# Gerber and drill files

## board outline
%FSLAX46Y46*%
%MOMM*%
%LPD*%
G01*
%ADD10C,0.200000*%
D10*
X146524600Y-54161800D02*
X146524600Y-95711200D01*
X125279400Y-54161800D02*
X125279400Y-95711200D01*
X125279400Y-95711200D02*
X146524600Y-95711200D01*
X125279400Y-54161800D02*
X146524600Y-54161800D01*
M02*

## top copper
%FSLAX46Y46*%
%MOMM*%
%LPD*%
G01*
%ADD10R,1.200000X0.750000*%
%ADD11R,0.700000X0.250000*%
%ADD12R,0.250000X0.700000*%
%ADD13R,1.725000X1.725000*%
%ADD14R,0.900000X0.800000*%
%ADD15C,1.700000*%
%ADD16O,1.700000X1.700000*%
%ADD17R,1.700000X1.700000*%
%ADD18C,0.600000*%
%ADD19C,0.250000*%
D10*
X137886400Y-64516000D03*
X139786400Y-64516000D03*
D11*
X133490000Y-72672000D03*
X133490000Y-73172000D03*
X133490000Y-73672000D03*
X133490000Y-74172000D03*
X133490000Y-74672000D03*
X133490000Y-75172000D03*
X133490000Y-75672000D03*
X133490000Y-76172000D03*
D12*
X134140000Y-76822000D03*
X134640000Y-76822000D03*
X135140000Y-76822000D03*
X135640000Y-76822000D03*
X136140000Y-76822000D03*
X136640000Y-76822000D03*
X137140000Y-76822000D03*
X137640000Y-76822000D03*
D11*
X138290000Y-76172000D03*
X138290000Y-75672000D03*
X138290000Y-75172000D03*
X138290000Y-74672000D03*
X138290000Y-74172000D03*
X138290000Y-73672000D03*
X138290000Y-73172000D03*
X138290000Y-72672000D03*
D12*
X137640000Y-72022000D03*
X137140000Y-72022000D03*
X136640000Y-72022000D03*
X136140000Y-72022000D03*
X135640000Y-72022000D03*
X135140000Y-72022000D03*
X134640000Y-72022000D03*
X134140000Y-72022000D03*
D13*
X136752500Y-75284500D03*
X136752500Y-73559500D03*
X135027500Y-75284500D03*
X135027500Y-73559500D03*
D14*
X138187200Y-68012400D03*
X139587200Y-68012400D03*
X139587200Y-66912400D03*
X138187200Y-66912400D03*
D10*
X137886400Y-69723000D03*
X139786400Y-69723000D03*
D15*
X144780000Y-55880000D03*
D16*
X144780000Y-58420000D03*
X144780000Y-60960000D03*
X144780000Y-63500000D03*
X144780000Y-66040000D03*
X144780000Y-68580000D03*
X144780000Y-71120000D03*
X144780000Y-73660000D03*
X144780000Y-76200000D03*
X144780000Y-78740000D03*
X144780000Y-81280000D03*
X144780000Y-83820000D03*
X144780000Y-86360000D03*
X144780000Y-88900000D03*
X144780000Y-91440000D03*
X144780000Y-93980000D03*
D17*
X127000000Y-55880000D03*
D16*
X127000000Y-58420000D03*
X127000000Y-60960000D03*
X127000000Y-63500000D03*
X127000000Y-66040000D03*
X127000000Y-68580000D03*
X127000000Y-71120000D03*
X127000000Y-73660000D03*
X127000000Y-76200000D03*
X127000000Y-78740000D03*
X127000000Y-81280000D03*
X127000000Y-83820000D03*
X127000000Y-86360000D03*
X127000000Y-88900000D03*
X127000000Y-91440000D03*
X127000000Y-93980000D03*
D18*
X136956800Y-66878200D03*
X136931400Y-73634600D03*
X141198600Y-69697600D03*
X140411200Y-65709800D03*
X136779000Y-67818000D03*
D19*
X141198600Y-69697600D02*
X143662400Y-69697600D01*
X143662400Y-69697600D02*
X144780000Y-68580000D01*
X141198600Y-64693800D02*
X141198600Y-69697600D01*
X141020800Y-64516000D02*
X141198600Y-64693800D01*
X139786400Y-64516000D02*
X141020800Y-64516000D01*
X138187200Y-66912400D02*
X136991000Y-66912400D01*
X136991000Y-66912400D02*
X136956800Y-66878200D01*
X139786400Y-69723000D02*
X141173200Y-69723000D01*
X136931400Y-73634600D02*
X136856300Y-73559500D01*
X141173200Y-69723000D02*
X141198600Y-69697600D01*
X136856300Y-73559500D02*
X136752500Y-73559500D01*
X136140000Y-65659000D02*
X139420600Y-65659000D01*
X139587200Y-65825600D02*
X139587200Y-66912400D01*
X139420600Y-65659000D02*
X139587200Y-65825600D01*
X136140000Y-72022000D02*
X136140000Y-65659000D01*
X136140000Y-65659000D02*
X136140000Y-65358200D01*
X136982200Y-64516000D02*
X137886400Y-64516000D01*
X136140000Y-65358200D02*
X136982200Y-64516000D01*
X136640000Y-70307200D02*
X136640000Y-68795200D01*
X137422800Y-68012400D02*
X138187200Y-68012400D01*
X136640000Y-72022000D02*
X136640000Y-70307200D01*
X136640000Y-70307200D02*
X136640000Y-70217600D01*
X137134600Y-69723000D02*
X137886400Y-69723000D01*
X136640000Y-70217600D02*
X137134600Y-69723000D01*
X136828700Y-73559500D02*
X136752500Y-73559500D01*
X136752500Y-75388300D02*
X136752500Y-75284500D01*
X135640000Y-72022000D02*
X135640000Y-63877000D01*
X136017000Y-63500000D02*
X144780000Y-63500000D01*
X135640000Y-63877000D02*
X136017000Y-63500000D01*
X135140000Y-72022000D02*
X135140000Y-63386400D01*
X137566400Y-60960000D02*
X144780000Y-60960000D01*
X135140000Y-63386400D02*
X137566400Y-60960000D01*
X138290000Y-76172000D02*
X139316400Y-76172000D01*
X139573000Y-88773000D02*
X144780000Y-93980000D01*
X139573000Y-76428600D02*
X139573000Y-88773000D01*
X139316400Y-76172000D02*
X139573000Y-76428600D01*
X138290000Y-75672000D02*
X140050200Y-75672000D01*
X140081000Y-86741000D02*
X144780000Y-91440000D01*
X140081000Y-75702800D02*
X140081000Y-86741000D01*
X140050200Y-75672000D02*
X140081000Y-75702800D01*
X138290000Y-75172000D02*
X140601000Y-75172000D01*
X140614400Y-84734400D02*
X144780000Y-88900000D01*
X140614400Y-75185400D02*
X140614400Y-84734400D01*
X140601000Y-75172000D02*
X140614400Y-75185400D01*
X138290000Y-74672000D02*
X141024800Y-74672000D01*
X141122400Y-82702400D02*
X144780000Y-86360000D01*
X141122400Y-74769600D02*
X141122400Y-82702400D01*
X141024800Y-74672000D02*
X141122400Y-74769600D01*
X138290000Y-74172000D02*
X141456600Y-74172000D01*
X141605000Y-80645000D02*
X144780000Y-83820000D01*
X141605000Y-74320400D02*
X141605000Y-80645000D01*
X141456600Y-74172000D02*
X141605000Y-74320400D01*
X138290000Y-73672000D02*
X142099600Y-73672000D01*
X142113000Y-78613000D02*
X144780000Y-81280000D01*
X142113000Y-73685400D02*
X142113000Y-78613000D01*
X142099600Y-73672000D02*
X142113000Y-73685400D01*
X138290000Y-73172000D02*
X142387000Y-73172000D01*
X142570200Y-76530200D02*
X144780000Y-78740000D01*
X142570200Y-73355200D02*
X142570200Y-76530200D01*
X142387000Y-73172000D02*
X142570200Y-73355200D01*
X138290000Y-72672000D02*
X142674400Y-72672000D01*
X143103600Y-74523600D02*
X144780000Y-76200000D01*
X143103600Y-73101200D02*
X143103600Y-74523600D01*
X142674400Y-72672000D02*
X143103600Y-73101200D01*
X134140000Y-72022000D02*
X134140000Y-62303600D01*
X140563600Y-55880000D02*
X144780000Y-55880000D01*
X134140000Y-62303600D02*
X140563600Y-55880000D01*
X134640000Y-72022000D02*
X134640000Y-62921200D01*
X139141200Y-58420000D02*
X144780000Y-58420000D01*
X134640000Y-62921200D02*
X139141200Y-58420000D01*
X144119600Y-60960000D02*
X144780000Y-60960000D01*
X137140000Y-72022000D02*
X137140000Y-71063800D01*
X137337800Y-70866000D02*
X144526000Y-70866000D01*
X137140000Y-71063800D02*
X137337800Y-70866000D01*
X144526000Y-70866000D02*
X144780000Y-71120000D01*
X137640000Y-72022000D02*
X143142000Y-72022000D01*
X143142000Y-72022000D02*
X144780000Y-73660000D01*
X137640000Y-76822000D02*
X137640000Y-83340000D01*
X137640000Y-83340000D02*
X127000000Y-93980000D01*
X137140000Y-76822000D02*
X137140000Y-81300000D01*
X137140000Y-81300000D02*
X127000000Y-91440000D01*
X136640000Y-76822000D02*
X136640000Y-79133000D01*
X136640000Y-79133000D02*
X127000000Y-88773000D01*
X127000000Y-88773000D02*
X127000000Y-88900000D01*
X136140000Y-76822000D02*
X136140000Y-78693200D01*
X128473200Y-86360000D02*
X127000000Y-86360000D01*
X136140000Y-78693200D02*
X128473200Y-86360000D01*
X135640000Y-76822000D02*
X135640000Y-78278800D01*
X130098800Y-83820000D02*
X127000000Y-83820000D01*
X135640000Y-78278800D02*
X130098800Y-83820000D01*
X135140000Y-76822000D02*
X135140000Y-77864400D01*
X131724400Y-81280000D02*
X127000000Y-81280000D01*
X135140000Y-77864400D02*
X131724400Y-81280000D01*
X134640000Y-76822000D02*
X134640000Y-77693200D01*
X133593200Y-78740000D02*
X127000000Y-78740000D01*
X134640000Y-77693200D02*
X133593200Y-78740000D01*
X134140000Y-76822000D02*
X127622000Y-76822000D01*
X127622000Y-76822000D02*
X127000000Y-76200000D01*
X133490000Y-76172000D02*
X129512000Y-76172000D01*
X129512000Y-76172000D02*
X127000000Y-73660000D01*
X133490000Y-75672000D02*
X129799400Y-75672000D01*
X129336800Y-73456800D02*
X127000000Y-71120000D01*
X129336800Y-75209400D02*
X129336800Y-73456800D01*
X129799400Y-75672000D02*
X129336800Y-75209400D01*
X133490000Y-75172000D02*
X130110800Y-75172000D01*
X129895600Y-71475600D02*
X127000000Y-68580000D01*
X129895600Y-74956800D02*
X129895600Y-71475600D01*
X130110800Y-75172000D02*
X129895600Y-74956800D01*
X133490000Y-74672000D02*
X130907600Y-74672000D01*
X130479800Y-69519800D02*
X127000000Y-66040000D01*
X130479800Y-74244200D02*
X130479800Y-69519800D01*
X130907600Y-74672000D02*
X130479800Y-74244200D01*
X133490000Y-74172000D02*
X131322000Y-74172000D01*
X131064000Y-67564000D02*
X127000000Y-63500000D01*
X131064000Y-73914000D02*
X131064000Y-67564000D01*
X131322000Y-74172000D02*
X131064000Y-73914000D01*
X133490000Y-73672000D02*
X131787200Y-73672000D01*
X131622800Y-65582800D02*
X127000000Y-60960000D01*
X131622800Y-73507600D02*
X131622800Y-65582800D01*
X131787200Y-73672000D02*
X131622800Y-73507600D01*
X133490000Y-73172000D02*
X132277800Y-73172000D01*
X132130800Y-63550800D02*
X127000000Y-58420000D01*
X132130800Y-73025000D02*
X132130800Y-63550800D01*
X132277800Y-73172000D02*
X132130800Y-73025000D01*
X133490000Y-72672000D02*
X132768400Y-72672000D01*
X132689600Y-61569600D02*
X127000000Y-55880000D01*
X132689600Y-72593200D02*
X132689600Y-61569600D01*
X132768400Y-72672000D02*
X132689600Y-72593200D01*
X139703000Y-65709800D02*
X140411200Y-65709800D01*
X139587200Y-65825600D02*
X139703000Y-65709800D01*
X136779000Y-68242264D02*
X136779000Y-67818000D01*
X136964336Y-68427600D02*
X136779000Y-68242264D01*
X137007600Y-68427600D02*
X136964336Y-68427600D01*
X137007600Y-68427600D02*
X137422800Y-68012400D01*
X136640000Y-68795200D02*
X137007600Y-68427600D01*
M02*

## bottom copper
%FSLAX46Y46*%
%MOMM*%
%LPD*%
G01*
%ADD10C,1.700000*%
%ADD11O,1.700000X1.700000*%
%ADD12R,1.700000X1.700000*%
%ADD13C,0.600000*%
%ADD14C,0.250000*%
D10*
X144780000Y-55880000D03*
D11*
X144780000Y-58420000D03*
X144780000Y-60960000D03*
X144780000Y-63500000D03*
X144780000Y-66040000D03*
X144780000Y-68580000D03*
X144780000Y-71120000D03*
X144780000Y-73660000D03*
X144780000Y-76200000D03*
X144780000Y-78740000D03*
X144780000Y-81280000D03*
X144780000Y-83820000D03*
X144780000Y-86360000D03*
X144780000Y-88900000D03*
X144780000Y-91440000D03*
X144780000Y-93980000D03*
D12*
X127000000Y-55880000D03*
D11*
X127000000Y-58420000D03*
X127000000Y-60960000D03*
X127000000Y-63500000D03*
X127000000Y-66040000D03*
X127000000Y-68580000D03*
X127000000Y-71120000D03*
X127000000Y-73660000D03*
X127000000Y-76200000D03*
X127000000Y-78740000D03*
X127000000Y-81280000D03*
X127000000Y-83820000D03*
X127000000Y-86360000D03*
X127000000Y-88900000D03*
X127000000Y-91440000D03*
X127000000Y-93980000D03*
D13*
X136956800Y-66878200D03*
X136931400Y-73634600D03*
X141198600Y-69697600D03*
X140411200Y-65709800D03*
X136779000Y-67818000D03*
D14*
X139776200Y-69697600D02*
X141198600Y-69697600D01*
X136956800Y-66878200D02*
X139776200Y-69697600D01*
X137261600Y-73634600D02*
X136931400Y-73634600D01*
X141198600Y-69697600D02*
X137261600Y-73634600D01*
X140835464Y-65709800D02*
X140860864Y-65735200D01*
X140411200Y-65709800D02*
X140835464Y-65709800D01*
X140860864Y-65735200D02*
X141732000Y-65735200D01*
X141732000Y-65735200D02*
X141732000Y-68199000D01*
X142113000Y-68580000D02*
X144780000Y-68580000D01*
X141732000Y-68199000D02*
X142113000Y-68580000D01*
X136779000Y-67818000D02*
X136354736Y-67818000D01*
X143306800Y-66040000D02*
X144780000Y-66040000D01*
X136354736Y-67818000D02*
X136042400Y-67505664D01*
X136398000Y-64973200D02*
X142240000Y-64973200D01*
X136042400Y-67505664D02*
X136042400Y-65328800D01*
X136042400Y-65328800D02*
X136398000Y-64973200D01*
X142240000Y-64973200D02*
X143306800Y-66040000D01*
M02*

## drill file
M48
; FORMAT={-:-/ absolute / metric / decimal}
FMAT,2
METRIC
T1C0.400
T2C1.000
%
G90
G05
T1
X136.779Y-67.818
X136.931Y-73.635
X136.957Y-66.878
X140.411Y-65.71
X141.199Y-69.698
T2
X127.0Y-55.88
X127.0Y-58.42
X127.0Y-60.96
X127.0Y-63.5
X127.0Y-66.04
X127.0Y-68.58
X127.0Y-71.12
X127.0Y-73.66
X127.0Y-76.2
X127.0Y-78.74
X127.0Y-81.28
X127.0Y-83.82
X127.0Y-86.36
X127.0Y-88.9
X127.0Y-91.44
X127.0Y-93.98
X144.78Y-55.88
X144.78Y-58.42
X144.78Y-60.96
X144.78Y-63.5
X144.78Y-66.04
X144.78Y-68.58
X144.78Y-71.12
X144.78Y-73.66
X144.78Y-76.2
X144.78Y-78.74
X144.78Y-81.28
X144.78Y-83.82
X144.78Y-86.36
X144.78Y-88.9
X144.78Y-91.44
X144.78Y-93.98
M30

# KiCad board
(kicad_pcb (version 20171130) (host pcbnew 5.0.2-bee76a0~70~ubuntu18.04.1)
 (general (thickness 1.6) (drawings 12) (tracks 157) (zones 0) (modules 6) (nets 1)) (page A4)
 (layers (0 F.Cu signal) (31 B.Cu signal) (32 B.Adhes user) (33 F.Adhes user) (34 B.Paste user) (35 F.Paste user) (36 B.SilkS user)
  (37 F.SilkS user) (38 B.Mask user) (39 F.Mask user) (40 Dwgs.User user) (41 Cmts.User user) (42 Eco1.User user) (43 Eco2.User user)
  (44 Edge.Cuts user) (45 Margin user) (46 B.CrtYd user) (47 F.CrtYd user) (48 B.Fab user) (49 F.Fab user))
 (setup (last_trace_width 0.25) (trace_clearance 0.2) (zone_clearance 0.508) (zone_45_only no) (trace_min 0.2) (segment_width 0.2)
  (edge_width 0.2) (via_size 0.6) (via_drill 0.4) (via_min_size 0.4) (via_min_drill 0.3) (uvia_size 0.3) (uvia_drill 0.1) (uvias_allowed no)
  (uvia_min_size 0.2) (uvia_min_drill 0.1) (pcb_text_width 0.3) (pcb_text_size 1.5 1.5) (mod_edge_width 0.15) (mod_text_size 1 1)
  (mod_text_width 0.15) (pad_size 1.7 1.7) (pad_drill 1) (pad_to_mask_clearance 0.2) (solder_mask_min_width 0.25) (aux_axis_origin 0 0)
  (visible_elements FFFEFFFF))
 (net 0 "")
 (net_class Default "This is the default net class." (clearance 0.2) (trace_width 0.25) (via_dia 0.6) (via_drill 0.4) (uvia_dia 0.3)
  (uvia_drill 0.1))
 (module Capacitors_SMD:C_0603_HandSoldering (layer F.Cu) (at 138.8364 64.516)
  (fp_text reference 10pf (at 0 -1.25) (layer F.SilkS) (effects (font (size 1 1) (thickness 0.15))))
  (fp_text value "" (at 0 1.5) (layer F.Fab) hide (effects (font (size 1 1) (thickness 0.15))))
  (pad 1 smd rect (at -0.95 0) (size 1.2 0.75) (layers F.Cu F.Paste F.Mask))
  (pad 2 smd rect (at 0.95 0) (size 1.2 0.75) (layers F.Cu F.Paste F.Mask)))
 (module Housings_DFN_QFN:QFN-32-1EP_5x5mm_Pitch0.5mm (layer F.Cu) (at 135.89 74.422)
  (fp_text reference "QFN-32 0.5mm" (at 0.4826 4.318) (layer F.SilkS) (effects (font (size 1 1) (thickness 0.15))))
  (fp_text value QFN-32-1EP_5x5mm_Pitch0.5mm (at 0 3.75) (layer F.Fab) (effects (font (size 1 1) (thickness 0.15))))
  (pad 1 smd rect (at -2.4 -1.75) (size 0.7 0.25) (layers F.Cu F.Paste F.Mask))
  (pad 2 smd rect (at -2.4 -1.25) (size 0.7 0.25) (layers F.Cu F.Paste F.Mask))
  (pad 3 smd rect (at -2.4 -0.75) (size 0.7 0.25) (layers F.Cu F.Paste F.Mask))
  (pad 4 smd rect (at -2.4 -0.25) (size 0.7 0.25) (layers F.Cu F.Paste F.Mask))
  (pad 5 smd rect (at -2.4 0.25) (size 0.7 0.25) (layers F.Cu F.Paste F.Mask))
  (pad 6 smd rect (at -2.4 0.75) (size 0.7 0.25) (layers F.Cu F.Paste F.Mask))
  (pad 7 smd rect (at -2.4 1.25) (size 0.7 0.25) (layers F.Cu F.Paste F.Mask))
  (pad 8 smd rect (at -2.4 1.75) (size 0.7 0.25) (layers F.Cu F.Paste F.Mask))
  (pad 9 smd rect (at -1.75 2.4 90) (size 0.7 0.25) (layers F.Cu F.Paste F.Mask))
  (pad 10 smd rect (at -1.25 2.4 90) (size 0.7 0.25) (layers F.Cu F.Paste F.Mask))
  (pad 11 smd rect (at -0.75 2.4 90) (size 0.7 0.25) (layers F.Cu F.Paste F.Mask))
  (pad 12 smd rect (at -0.25 2.4 90) (size 0.7 0.25) (layers F.Cu F.Paste F.Mask))
  (pad 13 smd rect (at 0.25 2.4 90) (size 0.7 0.25) (layers F.Cu F.Paste F.Mask))
  (pad 14 smd rect (at 0.75 2.4 90) (size 0.7 0.25) (layers F.Cu F.Paste F.Mask))
  (pad 15 smd rect (at 1.25 2.4 90) (size 0.7 0.25) (layers F.Cu F.Paste F.Mask))
  (pad 16 smd rect (at 1.75 2.4 90) (size 0.7 0.25) (layers F.Cu F.Paste F.Mask))
  (pad 17 smd rect (at 2.4 1.75) (size 0.7 0.25) (layers F.Cu F.Paste F.Mask))
  (pad 18 smd rect (at 2.4 1.25) (size 0.7 0.25) (layers F.Cu F.Paste F.Mask))
  (pad 19 smd rect (at 2.4 0.75) (size 0.7 0.25) (layers F.Cu F.Paste F.Mask))
  (pad 20 smd rect (at 2.4 0.25) (size 0.7 0.25) (layers F.Cu F.Paste F.Mask))
  (pad 21 smd rect (at 2.4 -0.25) (size 0.7 0.25) (layers F.Cu F.Paste F.Mask))
  (pad 22 smd rect (at 2.4 -0.75) (size 0.7 0.25) (layers F.Cu F.Paste F.Mask))
  (pad 23 smd rect (at 2.4 -1.25) (size 0.7 0.25) (layers F.Cu F.Paste F.Mask))
  (pad 24 smd rect (at 2.4 -1.75) (size 0.7 0.25) (layers F.Cu F.Paste F.Mask))
  (pad 25 smd rect (at 1.75 -2.4 90) (size 0.7 0.25) (layers F.Cu F.Paste F.Mask))
  (pad 26 smd rect (at 1.25 -2.4 90) (size 0.7 0.25) (layers F.Cu F.Paste F.Mask))
  (pad 27 smd rect (at 0.75 -2.4 90) (size 0.7 0.25) (layers F.Cu F.Paste F.Mask))
  (pad 28 smd rect (at 0.25 -2.4 90) (size 0.7 0.25) (layers F.Cu F.Paste F.Mask))
  (pad 29 smd rect (at -0.25 -2.4 90) (size 0.7 0.25) (layers F.Cu F.Paste F.Mask))
  (pad 30 smd rect (at -0.75 -2.4 90) (size 0.7 0.25) (layers F.Cu F.Paste F.Mask))
  (pad 31 smd rect (at -1.25 -2.4 90) (size 0.7 0.25) (layers F.Cu F.Paste F.Mask))
  (pad 32 smd rect (at -1.75 -2.4 90) (size 0.7 0.25) (layers F.Cu F.Paste F.Mask))
  (pad 33 smd rect (at 0.8625 0.8625) (size 1.725 1.725) (layers F.Cu F.Paste F.Mask) (solder_paste_margin_ratio -0.2))
  (pad 33 smd rect (at 0.8625 -0.8625) (size 1.725 1.725) (layers F.Cu F.Paste F.Mask) (solder_paste_margin_ratio -0.2))
  (pad 33 smd rect (at -0.8625 0.8625) (size 1.725 1.725) (layers F.Cu F.Paste F.Mask) (solder_paste_margin_ratio -0.2))
  (pad 33 smd rect (at -0.8625 -0.8625) (size 1.725 1.725) (layers F.Cu F.Paste F.Mask) (solder_paste_margin_ratio -0.2)))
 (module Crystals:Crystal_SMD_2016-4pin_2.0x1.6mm (layer F.Cu) (at 138.8872 67.4624)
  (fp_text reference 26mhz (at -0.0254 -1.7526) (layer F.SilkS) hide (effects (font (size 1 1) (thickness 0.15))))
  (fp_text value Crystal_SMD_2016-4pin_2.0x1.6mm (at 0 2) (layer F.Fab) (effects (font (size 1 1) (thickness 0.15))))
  (pad 1 smd rect (at -0.7 0.55) (size 0.9 0.8) (layers F.Cu F.Mask))
  (pad 2 smd rect (at 0.7 0.55) (size 0.9 0.8) (layers F.Cu F.Mask))
  (pad 3 smd rect (at 0.7 -0.55) (size 0.9 0.8) (layers F.Cu F.Mask))
  (pad 4 smd rect (at -0.7 -0.55) (size 0.9 0.8) (layers F.Cu F.Mask)))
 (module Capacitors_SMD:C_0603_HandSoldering (layer F.Cu) (at 138.8364 69.723)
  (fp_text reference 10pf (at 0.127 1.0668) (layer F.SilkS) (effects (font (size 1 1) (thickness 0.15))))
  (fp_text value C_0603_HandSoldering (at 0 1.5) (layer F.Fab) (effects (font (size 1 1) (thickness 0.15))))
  (pad 1 smd rect (at -0.95 0) (size 1.2 0.75) (layers F.Cu F.Paste F.Mask))
  (pad 2 smd rect (at 0.95 0) (size 1.2 0.75) (layers F.Cu F.Paste F.Mask)))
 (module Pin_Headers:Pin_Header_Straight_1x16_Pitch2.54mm (layer F.Cu) (at 144.78 55.88)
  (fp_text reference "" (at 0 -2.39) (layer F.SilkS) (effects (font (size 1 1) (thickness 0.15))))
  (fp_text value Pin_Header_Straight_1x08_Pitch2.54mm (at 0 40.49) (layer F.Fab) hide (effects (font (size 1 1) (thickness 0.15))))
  (pad 1 thru_hole circle (at 0 0) (size 1.7 1.7) (drill 1) (layers *.Cu *.Mask))
  (pad 2 thru_hole oval (at 0 2.54) (size 1.7 1.7) (drill 1) (layers *.Cu *.Mask))
  (pad 3 thru_hole oval (at 0 5.08) (size 1.7 1.7) (drill 1) (layers *.Cu *.Mask))
  (pad 4 thru_hole oval (at 0 7.62) (size 1.7 1.7) (drill 1) (layers *.Cu *.Mask))
  (pad 5 thru_hole oval (at 0 10.16) (size 1.7 1.7) (drill 1) (layers *.Cu *.Mask))
  (pad 6 thru_hole oval (at 0 12.7) (size 1.7 1.7) (drill 1) (layers *.Cu *.Mask))
  (pad 7 thru_hole oval (at 0 15.24) (size 1.7 1.7) (drill 1) (layers *.Cu *.Mask))
  (pad 8 thru_hole oval (at 0 17.78) (size 1.7 1.7) (drill 1) (layers *.Cu *.Mask))
  (pad 9 thru_hole oval (at 0 20.32) (size 1.7 1.7) (drill 1) (layers *.Cu *.Mask))
  (pad 10 thru_hole oval (at 0 22.86) (size 1.7 1.7) (drill 1) (layers *.Cu *.Mask))
  (pad 11 thru_hole oval (at 0 25.4) (size 1.7 1.7) (drill 1) (layers *.Cu *.Mask))
  (pad 12 thru_hole oval (at 0 27.94) (size 1.7 1.7) (drill 1) (layers *.Cu *.Mask))
  (pad 13 thru_hole oval (at 0 30.48) (size 1.7 1.7) (drill 1) (layers *.Cu *.Mask))
  (pad 14 thru_hole oval (at 0 33.02) (size 1.7 1.7) (drill 1) (layers *.Cu *.Mask))
  (pad 15 thru_hole oval (at 0 35.56) (size 1.7 1.7) (drill 1) (layers *.Cu *.Mask))
  (pad 16 thru_hole oval (at 0 38.1) (size 1.7 1.7) (drill 1) (layers *.Cu *.Mask)))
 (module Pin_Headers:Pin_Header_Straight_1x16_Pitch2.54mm (layer F.Cu) (at 127 55.88)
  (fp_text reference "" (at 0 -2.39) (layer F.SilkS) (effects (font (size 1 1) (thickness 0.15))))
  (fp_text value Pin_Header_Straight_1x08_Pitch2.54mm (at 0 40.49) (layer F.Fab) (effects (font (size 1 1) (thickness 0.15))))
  (pad 1 thru_hole rect (at 0 0) (size 1.7 1.7) (drill 1) (layers *.Cu *.Mask))
  (pad 2 thru_hole oval (at 0 2.54) (size 1.7 1.7) (drill 1) (layers *.Cu *.Mask))
  (pad 3 thru_hole oval (at 0 5.08) (size 1.7 1.7) (drill 1) (layers *.Cu *.Mask))
  (pad 4 thru_hole oval (at 0 7.62) (size 1.7 1.7) (drill 1) (layers *.Cu *.Mask))
  (pad 5 thru_hole oval (at 0 10.16) (size 1.7 1.7) (drill 1) (layers *.Cu *.Mask))
  (pad 6 thru_hole oval (at 0 12.7) (size 1.7 1.7) (drill 1) (layers *.Cu *.Mask))
  (pad 7 thru_hole oval (at 0 15.24) (size 1.7 1.7) (drill 1) (layers *.Cu *.Mask))
  (pad 8 thru_hole oval (at 0 17.78) (size 1.7 1.7) (drill 1) (layers *.Cu *.Mask))
  (pad 9 thru_hole oval (at 0 20.32) (size 1.7 1.7) (drill 1) (layers *.Cu *.Mask))
  (pad 10 thru_hole oval (at 0 22.86) (size 1.7 1.7) (drill 1) (layers *.Cu *.Mask))
  (pad 11 thru_hole oval (at 0 25.4) (size 1.7 1.7) (drill 1) (layers *.Cu *.Mask))
  (pad 12 thru_hole oval (at 0 27.94) (size 1.7 1.7) (drill 1) (layers *.Cu *.Mask))
  (pad 13 thru_hole oval (at 0 30.48) (size 1.7 1.7) (drill 1) (layers *.Cu *.Mask))
  (pad 14 thru_hole oval (at 0 33.02) (size 1.7 1.7) (drill 1) (layers *.Cu *.Mask))
  (pad 15 thru_hole oval (at 0 35.56) (size 1.7 1.7) (drill 1) (layers *.Cu *.Mask))
  (pad 16 thru_hole oval (at 0 38.1) (size 1.7 1.7) (drill 1) (layers *.Cu *.Mask)))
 (gr_line (start 146.5246 54.1618) (end 146.5246 95.7112) (angle 90) (layer Edge.Cuts) (width 0.2))
 (gr_line (start 125.2794 54.1618) (end 125.2794 95.7112) (angle 90) (layer Edge.Cuts) (width 0.2))
 (gr_line (start 125.2794 95.7112) (end 146.5246 95.7112) (angle 90) (layer Edge.Cuts) (width 0.2))
 (gr_line (start 125.2794 54.1618) (end 146.5246 54.1618) (angle 90) (layer Edge.Cuts) (width 0.2))
 (segment (start 141.1986 69.6976) (end 143.6624 69.6976) (width 0.25) (layer F.Cu) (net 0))
 (segment (start 143.6624 69.6976) (end 144.78 68.58) (width 0.25) (layer F.Cu) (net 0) (status 800000))
 (segment (start 141.1986 64.6938) (end 141.1986 69.6976) (width 0.25) (layer F.Cu) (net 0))
 (segment (start 141.0208 64.516) (end 141.1986 64.6938) (width 0.25) (layer F.Cu) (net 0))
 (segment (start 139.7864 64.516) (end 141.0208 64.516) (width 0.25) (layer F.Cu) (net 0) (status 10))
 (segment (start 138.1872 66.9124) (end 136.991 66.9124) (width 0.25) (layer F.Cu) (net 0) (status 10))
 (segment (start 139.7762 69.6976) (end 141.1986 69.6976) (width 0.25) (layer B.Cu) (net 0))
 (segment (start 136.9568 66.8782) (end 139.7762 69.6976) (width 0.25) (layer B.Cu) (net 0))
 (via (at 136.9568 66.8782) (size 0.6) (drill 0.4) (layers F.Cu B.Cu) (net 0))
 (segment (start 136.991 66.9124) (end 136.9568 66.8782) (width 0.25) (layer F.Cu) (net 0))
 (segment (start 139.7864 69.723) (end 141.1732 69.723) (width 0.25) (layer F.Cu) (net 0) (status 10))
 (segment (start 136.9314 73.6346) (end 136.8563 73.5595) (width 0.25) (layer F.Cu) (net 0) (status 30))
 (via (at 136.9314 73.6346) (size 0.6) (drill 0.4) (layers F.Cu B.Cu) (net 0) (status 30))
 (segment (start 137.2616 73.6346) (end 136.9314 73.6346) (width 0.25) (layer B.Cu) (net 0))
 (segment (start 141.1986 69.6976) (end 137.2616 73.6346) (width 0.25) (layer B.Cu) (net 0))
 (via (at 141.1986 69.6976) (size 0.6) (drill 0.4) (layers F.Cu B.Cu) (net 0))
 (segment (start 141.1732 69.723) (end 141.1986 69.6976) (width 0.25) (layer F.Cu) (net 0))
 (segment (start 136.8563 73.5595) (end 136.7525 73.5595) (width 0.25) (layer F.Cu) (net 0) (status 30))
 (segment (start 136.14 65.659) (end 139.4206 65.659) (width 0.25) (layer F.Cu) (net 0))
 (segment (start 139.5872 65.8256) (end 139.5872 66.9124) (width 0.25) (layer F.Cu) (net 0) (status 20))
 (segment (start 139.4206 65.659) (end 139.5872 65.8256) (width 0.25) (layer F.Cu) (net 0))
 (segment (start 136.14 72.022) (end 136.14 65.659) (width 0.25) (layer F.Cu) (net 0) (status 10))
 (segment (start 136.14 65.659) (end 136.14 65.3582) (width 0.25) (layer F.Cu) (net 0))
 (segment (start 136.9822 64.516) (end 137.8864 64.516) (width 0.25) (layer F.Cu) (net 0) (status 20))
 (segment (start 136.14 65.3582) (end 136.9822 64.516) (width 0.25) (layer F.Cu) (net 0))
 (segment (start 136.64 70.3072) (end 136.64 68.7952) (width 0.25) (layer F.Cu) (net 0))
 (segment (start 137.4228 68.0124) (end 138.1872 68.0124) (width 0.25) (layer F.Cu) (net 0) (status 20))
 (segment (start 136.64 72.022) (end 136.64 70.3072) (width 0.25) (layer F.Cu) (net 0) (status 10))
 (segment (start 136.64 70.3072) (end 136.64 70.2176) (width 0.25) (layer F.Cu) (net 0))
 (segment (start 137.1346 69.723) (end 137.8864 69.723) (width 0.25) (layer F.Cu) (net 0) (status 20))
 (segment (start 136.64 70.2176) (end 137.1346 69.723) (width 0.25) (layer F.Cu) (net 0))
 (segment (start 136.8287 73.5595) (end 136.7525 73.5595) (width 0.25) (layer F.Cu) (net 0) (status 30))
 (segment (start 136.7525 75.3883) (end 136.7525 75.2845) (width 0.25) (layer F.Cu) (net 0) (status 30))
 (segment (start 135.64 72.022) (end 135.64 63.877) (width 0.25) (layer F.Cu) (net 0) (status 10))
 (segment (start 136.017 63.5) (end 144.78 63.5) (width 0.25) (layer F.Cu) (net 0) (status 20))
 (segment (start 135.64 63.877) (end 136.017 63.5) (width 0.25) (layer F.Cu) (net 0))
 (segment (start 135.14 72.022) (end 135.14 63.3864) (width 0.25) (layer F.Cu) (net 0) (status 10))
 (segment (start 137.5664 60.96) (end 144.78 60.96) (width 0.25) (layer F.Cu) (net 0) (status 20))
 (segment (start 135.14 63.3864) (end 137.5664 60.96) (width 0.25) (layer F.Cu) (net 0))
 (segment (start 138.29 76.172) (end 139.3164 76.172) (width 0.25) (layer F.Cu) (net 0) (status 10))
 (segment (start 139.573 88.773) (end 144.78 93.98) (width 0.25) (layer F.Cu) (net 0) (status 20))
 (segment (start 139.573 76.4286) (end 139.573 88.773) (width 0.25) (layer F.Cu) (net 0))
 (segment (start 139.3164 76.172) (end 139.573 76.4286) (width 0.25) (layer F.Cu) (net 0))
 (segment (start 138.29 75.672) (end 140.0502 75.672) (width 0.25) (layer F.Cu) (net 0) (status 10))
 (segment (start 140.081 86.741) (end 144.78 91.44) (width 0.25) (layer F.Cu) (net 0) (status 20))
 (segment (start 140.081 75.7028) (end 140.081 86.741) (width 0.25) (layer F.Cu) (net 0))
 (segment (start 140.0502 75.672) (end 140.081 75.7028) (width 0.25) (layer F.Cu) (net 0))
 (segment (start 138.29 75.172) (end 140.601 75.172) (width 0.25) (layer F.Cu) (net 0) (status 10))
 (segment (start 140.6144 84.7344) (end 144.78 88.9) (width 0.25) (layer F.Cu) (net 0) (status 20))
 (segment (start 140.6144 75.1854) (end 140.6144 84.7344) (width 0.25) (layer F.Cu) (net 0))
 (segment (start 140.601 75.172) (end 140.6144 75.1854) (width 0.25) (layer F.Cu) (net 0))
 (segment (start 138.29 74.672) (end 141.0248 74.672) (width 0.25) (layer F.Cu) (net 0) (status 10))
 (segment (start 141.1224 82.7024) (end 144.78 86.36) (width 0.25) (layer F.Cu) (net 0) (status 20))
 (segment (start 141.1224 74.7696) (end 141.1224 82.7024) (width 0.25) (layer F.Cu) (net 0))
 (segment (start 141.0248 74.672) (end 141.1224 74.7696) (width 0.25) (layer F.Cu) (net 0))
 (segment (start 138.29 74.172) (end 141.4566 74.172) (width 0.25) (layer F.Cu) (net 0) (status 10))
 (segment (start 141.605 80.645) (end 144.78 83.82) (width 0.25) (layer F.Cu) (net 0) (status 20))
 (segment (start 141.605 74.3204) (end 141.605 80.645) (width 0.25) (layer F.Cu) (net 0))
 (segment (start 141.4566 74.172) (end 141.605 74.3204) (width 0.25) (layer F.Cu) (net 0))
 (segment (start 138.29 73.672) (end 142.0996 73.672) (width 0.25) (layer F.Cu) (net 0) (status 10))
 (segment (start 142.113 78.613) (end 144.78 81.28) (width 0.25) (layer F.Cu) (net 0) (status 20))
 (segment (start 142.113 73.6854) (end 142.113 78.613) (width 0.25) (layer F.Cu) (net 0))
 (segment (start 142.0996 73.672) (end 142.113 73.6854) (width 0.25) (layer F.Cu) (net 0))
 (segment (start 138.29 73.172) (end 142.387 73.172) (width 0.25) (layer F.Cu) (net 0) (status 10))
 (segment (start 142.5702 76.5302) (end 144.78 78.74) (width 0.25) (layer F.Cu) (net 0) (status 20))
 (segment (start 142.5702 73.3552) (end 142.5702 76.5302) (width 0.25) (layer F.Cu) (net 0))
 (segment (start 142.387 73.172) (end 142.5702 73.3552) (width 0.25) (layer F.Cu) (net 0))
 (segment (start 138.29 72.672) (end 142.6744 72.672) (width 0.25) (layer F.Cu) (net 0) (status 10))
 (segment (start 143.1036 74.5236) (end 144.78 76.2) (width 0.25) (layer F.Cu) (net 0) (status 20))
 (segment (start 143.1036 73.1012) (end 143.1036 74.5236) (width 0.25) (layer F.Cu) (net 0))
 (segment (start 142.6744 72.672) (end 143.1036 73.1012) (width 0.25) (layer F.Cu) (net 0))
 (segment (start 134.14 72.022) (end 134.14 62.3036) (width 0.25) (layer F.Cu) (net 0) (status 10))
 (segment (start 140.5636 55.88) (end 144.78 55.88) (width 0.25) (layer F.Cu) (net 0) (status 20))
 (segment (start 134.14 62.3036) (end 140.5636 55.88) (width 0.25) (layer F.Cu) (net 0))
 (segment (start 134.64 72.022) (end 134.64 62.9212) (width 0.25) (layer F.Cu) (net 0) (status 10))
 (segment (start 139.1412 58.42) (end 144.78 58.42) (width 0.25) (layer F.Cu) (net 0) (status 20))
 (segment (start 134.64 62.9212) (end 139.1412 58.42) (width 0.25) (layer F.Cu) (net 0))
 (segment (start 144.1196 60.96) (end 144.78 60.96) (width 0.25) (layer F.Cu) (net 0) (status 30))
 (segment (start 137.14 72.022) (end 137.14 71.0638) (width 0.25) (layer F.Cu) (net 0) (status 10))
 (segment (start 137.3378 70.866) (end 144.526 70.866) (width 0.25) (layer F.Cu) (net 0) (status 20))
 (segment (start 137.14 71.0638) (end 137.3378 70.866) (width 0.25) (layer F.Cu) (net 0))
 (segment (start 144.526 70.866) (end 144.78 71.12) (width 0.25) (layer F.Cu) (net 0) (status 30))
 (segment (start 137.64 72.022) (end 143.142 72.022) (width 0.25) (layer F.Cu) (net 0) (status 10))
 (segment (start 143.142 72.022) (end 144.78 73.66) (width 0.25) (layer F.Cu) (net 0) (status 20))
 (segment (start 137.64 76.822) (end 137.64 83.34) (width 0.25) (layer F.Cu) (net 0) (status 10))
 (segment (start 137.64 83.34) (end 127 93.98) (width 0.25) (layer F.Cu) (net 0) (status 20))
 (segment (start 137.14 76.822) (end 137.14 81.3) (width 0.25) (layer F.Cu) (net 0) (status 10))
 (segment (start 137.14 81.3) (end 127 91.44) (width 0.25) (layer F.Cu) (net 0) (status 20))
 (segment (start 136.64 76.822) (end 136.64 79.133) (width 0.25) (layer F.Cu) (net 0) (status 10))
 (segment (start 136.64 79.133) (end 127 88.773) (width 0.25) (layer F.Cu) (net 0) (status 20))
 (segment (start 127 88.773) (end 127 88.9) (width 0.25) (layer F.Cu) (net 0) (status 30))
 (segment (start 136.14 76.822) (end 136.14 78.6932) (width 0.25) (layer F.Cu) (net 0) (status 10))
 (segment (start 128.4732 86.36) (end 127 86.36) (width 0.25) (layer F.Cu) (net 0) (status 20))
 (segment (start 136.14 78.6932) (end 128.4732 86.36) (width 0.25) (layer F.Cu) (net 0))
 (segment (start 135.64 76.822) (end 135.64 78.2788) (width 0.25) (layer F.Cu) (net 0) (status 10))
 (segment (start 130.0988 83.82) (end 127 83.82) (width 0.25) (layer F.Cu) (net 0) (status 20))
 (segment (start 135.64 78.2788) (end 130.0988 83.82) (width 0.25) (layer F.Cu) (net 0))
 (segment (start 135.14 76.822) (end 135.14 77.8644) (width 0.25) (layer F.Cu) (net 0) (status 10))
 (segment (start 131.7244 81.28) (end 127 81.28) (width 0.25) (layer F.Cu) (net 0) (status 20))
 (segment (start 135.14 77.8644) (end 131.7244 81.28) (width 0.25) (layer F.Cu) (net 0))
 (segment (start 134.64 76.822) (end 134.64 77.6932) (width 0.25) (layer F.Cu) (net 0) (status 10))
 (segment (start 133.5932 78.74) (end 127 78.74) (width 0.25) (layer F.Cu) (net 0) (status 20))
 (segment (start 134.64 77.6932) (end 133.5932 78.74) (width 0.25) (layer F.Cu) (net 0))
 (segment (start 134.14 76.822) (end 127.622 76.822) (width 0.25) (layer F.Cu) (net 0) (status 10))
 (segment (start 127.622 76.822) (end 127 76.2) (width 0.25) (layer F.Cu) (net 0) (status 20))
 (segment (start 133.49 76.172) (end 129.512 76.172) (width 0.25) (layer F.Cu) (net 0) (status 10))
 (segment (start 129.512 76.172) (end 127 73.66) (width 0.25) (layer F.Cu) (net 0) (status 20))
 (segment (start 133.49 75.672) (end 129.7994 75.672) (width 0.25) (layer F.Cu) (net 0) (status 10))
 (segment (start 129.3368 73.4568) (end 127 71.12) (width 0.25) (layer F.Cu) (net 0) (status 20))
 (segment (start 129.3368 75.2094) (end 129.3368 73.4568) (width 0.25) (layer F.Cu) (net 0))
 (segment (start 129.7994 75.672) (end 129.3368 75.2094) (width 0.25) (layer F.Cu) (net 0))
 (segment (start 133.49 75.172) (end 130.1108 75.172) (width 0.25) (layer F.Cu) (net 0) (status 10))
 (segment (start 129.8956 71.4756) (end 127 68.58) (width 0.25) (layer F.Cu) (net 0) (status 20))
 (segment (start 129.8956 74.9568) (end 129.8956 71.4756) (width 0.25) (layer F.Cu) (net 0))
 (segment (start 130.1108 75.172) (end 129.8956 74.9568) (width 0.25) (layer F.Cu) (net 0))
 (segment (start 133.49 74.672) (end 130.9076 74.672) (width 0.25) (layer F.Cu) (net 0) (status 10))
 (segment (start 130.4798 69.5198) (end 127 66.04) (width 0.25) (layer F.Cu) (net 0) (status 20))
 (segment (start 130.4798 74.2442) (end 130.4798 69.5198) (width 0.25) (layer F.Cu) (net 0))
 (segment (start 130.9076 74.672) (end 130.4798 74.2442) (width 0.25) (layer F.Cu) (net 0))
 (segment (start 133.49 74.172) (end 131.322 74.172) (width 0.25) (layer F.Cu) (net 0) (status 10))
 (segment (start 131.064 67.564) (end 127 63.5) (width 0.25) (layer F.Cu) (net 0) (status 20))
 (segment (start 131.064 73.914) (end 131.064 67.564) (width 0.25) (layer F.Cu) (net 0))
 (segment (start 131.322 74.172) (end 131.064 73.914) (width 0.25) (layer F.Cu) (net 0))
 (segment (start 133.49 73.672) (end 131.7872 73.672) (width 0.25) (layer F.Cu) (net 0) (status 10))
 (segment (start 131.6228 65.5828) (end 127 60.96) (width 0.25) (layer F.Cu) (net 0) (status 20))
 (segment (start 131.6228 73.5076) (end 131.6228 65.5828) (width 0.25) (layer F.Cu) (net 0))
 (segment (start 131.7872 73.672) (end 131.6228 73.5076) (width 0.25) (layer F.Cu) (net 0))
 (segment (start 133.49 73.172) (end 132.2778 73.172) (width 0.25) (layer F.Cu) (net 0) (status 10))
 (segment (start 132.1308 63.5508) (end 127 58.42) (width 0.25) (layer F.Cu) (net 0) (status 20))
 (segment (start 132.1308 73.025) (end 132.1308 63.5508) (width 0.25) (layer F.Cu) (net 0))
 (segment (start 132.2778 73.172) (end 132.1308 73.025) (width 0.25) (layer F.Cu) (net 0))
 (segment (start 133.49 72.672) (end 132.7684 72.672) (width 0.25) (layer F.Cu) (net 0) (status 10))
 (segment (start 132.6896 61.5696) (end 127 55.88) (width 0.25) (layer F.Cu) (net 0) (status 20))
 (segment (start 132.6896 72.5932) (end 132.6896 61.5696) (width 0.25) (layer F.Cu) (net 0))
 (segment (start 132.7684 72.672) (end 132.6896 72.5932) (width 0.25) (layer F.Cu) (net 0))
 (via (at 140.4112 65.7098) (size 0.6) (drill 0.4) (layers F.Cu B.Cu) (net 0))
 (via (at 136.779 67.818) (size 0.6) (drill 0.4) (layers F.Cu B.Cu) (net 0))
 (segment (start 139.703 65.7098) (end 140.4112 65.7098) (width 0.25) (layer F.Cu) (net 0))
 (segment (start 139.5872 65.8256) (end 139.703 65.7098) (width 0.25) (layer F.Cu) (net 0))
 (segment (start 136.779 68.242264) (end 136.779 67.818) (width 0.25) (layer F.Cu) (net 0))
 (segment (start 136.964336 68.4276) (end 136.779 68.242264) (width 0.25) (layer F.Cu) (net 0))
 (segment (start 137.0076 68.4276) (end 136.964336 68.4276) (width 0.25) (layer F.Cu) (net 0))
 (segment (start 137.0076 68.4276) (end 137.4228 68.0124) (width 0.25) (layer F.Cu) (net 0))
 (segment (start 136.64 68.7952) (end 137.0076 68.4276) (width 0.25) (layer F.Cu) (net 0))
 (segment (start 140.835464 65.7098) (end 140.860864 65.7352) (width 0.25) (layer B.Cu) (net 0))
 (segment (start 140.4112 65.7098) (end 140.835464 65.7098) (width 0.25) (layer B.Cu) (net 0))
 (segment (start 140.860864 65.7352) (end 141.732 65.7352) (width 0.25) (layer B.Cu) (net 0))
 (segment (start 141.732 65.7352) (end 141.732 68.199) (width 0.25) (layer B.Cu) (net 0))
 (segment (start 142.113 68.58) (end 144.78 68.58) (width 0.25) (layer B.Cu) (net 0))
 (segment (start 141.732 68.199) (end 142.113 68.58) (width 0.25) (layer B.Cu) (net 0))
 (segment (start 136.779 67.818) (end 136.354736 67.818) (width 0.25) (layer B.Cu) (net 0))
 (segment (start 143.3068 66.04) (end 144.78 66.04) (width 0.25) (layer B.Cu) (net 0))
 (segment (start 136.354736 67.818) (end 136.0424 67.505664) (width 0.25) (layer B.Cu) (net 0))
 (segment (start 136.398 64.9732) (end 142.24 64.9732) (width 0.25) (layer B.Cu) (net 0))
 (segment (start 136.0424 67.505664) (end 136.0424 65.3288) (width 0.25) (layer B.Cu) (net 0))
 (segment (start 136.0424 65.3288) (end 136.398 64.9732) (width 0.25) (layer B.Cu) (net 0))
 (segment (start 142.24 64.9732) (end 143.3068 66.04) (width 0.25) (layer B.Cu) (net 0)))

